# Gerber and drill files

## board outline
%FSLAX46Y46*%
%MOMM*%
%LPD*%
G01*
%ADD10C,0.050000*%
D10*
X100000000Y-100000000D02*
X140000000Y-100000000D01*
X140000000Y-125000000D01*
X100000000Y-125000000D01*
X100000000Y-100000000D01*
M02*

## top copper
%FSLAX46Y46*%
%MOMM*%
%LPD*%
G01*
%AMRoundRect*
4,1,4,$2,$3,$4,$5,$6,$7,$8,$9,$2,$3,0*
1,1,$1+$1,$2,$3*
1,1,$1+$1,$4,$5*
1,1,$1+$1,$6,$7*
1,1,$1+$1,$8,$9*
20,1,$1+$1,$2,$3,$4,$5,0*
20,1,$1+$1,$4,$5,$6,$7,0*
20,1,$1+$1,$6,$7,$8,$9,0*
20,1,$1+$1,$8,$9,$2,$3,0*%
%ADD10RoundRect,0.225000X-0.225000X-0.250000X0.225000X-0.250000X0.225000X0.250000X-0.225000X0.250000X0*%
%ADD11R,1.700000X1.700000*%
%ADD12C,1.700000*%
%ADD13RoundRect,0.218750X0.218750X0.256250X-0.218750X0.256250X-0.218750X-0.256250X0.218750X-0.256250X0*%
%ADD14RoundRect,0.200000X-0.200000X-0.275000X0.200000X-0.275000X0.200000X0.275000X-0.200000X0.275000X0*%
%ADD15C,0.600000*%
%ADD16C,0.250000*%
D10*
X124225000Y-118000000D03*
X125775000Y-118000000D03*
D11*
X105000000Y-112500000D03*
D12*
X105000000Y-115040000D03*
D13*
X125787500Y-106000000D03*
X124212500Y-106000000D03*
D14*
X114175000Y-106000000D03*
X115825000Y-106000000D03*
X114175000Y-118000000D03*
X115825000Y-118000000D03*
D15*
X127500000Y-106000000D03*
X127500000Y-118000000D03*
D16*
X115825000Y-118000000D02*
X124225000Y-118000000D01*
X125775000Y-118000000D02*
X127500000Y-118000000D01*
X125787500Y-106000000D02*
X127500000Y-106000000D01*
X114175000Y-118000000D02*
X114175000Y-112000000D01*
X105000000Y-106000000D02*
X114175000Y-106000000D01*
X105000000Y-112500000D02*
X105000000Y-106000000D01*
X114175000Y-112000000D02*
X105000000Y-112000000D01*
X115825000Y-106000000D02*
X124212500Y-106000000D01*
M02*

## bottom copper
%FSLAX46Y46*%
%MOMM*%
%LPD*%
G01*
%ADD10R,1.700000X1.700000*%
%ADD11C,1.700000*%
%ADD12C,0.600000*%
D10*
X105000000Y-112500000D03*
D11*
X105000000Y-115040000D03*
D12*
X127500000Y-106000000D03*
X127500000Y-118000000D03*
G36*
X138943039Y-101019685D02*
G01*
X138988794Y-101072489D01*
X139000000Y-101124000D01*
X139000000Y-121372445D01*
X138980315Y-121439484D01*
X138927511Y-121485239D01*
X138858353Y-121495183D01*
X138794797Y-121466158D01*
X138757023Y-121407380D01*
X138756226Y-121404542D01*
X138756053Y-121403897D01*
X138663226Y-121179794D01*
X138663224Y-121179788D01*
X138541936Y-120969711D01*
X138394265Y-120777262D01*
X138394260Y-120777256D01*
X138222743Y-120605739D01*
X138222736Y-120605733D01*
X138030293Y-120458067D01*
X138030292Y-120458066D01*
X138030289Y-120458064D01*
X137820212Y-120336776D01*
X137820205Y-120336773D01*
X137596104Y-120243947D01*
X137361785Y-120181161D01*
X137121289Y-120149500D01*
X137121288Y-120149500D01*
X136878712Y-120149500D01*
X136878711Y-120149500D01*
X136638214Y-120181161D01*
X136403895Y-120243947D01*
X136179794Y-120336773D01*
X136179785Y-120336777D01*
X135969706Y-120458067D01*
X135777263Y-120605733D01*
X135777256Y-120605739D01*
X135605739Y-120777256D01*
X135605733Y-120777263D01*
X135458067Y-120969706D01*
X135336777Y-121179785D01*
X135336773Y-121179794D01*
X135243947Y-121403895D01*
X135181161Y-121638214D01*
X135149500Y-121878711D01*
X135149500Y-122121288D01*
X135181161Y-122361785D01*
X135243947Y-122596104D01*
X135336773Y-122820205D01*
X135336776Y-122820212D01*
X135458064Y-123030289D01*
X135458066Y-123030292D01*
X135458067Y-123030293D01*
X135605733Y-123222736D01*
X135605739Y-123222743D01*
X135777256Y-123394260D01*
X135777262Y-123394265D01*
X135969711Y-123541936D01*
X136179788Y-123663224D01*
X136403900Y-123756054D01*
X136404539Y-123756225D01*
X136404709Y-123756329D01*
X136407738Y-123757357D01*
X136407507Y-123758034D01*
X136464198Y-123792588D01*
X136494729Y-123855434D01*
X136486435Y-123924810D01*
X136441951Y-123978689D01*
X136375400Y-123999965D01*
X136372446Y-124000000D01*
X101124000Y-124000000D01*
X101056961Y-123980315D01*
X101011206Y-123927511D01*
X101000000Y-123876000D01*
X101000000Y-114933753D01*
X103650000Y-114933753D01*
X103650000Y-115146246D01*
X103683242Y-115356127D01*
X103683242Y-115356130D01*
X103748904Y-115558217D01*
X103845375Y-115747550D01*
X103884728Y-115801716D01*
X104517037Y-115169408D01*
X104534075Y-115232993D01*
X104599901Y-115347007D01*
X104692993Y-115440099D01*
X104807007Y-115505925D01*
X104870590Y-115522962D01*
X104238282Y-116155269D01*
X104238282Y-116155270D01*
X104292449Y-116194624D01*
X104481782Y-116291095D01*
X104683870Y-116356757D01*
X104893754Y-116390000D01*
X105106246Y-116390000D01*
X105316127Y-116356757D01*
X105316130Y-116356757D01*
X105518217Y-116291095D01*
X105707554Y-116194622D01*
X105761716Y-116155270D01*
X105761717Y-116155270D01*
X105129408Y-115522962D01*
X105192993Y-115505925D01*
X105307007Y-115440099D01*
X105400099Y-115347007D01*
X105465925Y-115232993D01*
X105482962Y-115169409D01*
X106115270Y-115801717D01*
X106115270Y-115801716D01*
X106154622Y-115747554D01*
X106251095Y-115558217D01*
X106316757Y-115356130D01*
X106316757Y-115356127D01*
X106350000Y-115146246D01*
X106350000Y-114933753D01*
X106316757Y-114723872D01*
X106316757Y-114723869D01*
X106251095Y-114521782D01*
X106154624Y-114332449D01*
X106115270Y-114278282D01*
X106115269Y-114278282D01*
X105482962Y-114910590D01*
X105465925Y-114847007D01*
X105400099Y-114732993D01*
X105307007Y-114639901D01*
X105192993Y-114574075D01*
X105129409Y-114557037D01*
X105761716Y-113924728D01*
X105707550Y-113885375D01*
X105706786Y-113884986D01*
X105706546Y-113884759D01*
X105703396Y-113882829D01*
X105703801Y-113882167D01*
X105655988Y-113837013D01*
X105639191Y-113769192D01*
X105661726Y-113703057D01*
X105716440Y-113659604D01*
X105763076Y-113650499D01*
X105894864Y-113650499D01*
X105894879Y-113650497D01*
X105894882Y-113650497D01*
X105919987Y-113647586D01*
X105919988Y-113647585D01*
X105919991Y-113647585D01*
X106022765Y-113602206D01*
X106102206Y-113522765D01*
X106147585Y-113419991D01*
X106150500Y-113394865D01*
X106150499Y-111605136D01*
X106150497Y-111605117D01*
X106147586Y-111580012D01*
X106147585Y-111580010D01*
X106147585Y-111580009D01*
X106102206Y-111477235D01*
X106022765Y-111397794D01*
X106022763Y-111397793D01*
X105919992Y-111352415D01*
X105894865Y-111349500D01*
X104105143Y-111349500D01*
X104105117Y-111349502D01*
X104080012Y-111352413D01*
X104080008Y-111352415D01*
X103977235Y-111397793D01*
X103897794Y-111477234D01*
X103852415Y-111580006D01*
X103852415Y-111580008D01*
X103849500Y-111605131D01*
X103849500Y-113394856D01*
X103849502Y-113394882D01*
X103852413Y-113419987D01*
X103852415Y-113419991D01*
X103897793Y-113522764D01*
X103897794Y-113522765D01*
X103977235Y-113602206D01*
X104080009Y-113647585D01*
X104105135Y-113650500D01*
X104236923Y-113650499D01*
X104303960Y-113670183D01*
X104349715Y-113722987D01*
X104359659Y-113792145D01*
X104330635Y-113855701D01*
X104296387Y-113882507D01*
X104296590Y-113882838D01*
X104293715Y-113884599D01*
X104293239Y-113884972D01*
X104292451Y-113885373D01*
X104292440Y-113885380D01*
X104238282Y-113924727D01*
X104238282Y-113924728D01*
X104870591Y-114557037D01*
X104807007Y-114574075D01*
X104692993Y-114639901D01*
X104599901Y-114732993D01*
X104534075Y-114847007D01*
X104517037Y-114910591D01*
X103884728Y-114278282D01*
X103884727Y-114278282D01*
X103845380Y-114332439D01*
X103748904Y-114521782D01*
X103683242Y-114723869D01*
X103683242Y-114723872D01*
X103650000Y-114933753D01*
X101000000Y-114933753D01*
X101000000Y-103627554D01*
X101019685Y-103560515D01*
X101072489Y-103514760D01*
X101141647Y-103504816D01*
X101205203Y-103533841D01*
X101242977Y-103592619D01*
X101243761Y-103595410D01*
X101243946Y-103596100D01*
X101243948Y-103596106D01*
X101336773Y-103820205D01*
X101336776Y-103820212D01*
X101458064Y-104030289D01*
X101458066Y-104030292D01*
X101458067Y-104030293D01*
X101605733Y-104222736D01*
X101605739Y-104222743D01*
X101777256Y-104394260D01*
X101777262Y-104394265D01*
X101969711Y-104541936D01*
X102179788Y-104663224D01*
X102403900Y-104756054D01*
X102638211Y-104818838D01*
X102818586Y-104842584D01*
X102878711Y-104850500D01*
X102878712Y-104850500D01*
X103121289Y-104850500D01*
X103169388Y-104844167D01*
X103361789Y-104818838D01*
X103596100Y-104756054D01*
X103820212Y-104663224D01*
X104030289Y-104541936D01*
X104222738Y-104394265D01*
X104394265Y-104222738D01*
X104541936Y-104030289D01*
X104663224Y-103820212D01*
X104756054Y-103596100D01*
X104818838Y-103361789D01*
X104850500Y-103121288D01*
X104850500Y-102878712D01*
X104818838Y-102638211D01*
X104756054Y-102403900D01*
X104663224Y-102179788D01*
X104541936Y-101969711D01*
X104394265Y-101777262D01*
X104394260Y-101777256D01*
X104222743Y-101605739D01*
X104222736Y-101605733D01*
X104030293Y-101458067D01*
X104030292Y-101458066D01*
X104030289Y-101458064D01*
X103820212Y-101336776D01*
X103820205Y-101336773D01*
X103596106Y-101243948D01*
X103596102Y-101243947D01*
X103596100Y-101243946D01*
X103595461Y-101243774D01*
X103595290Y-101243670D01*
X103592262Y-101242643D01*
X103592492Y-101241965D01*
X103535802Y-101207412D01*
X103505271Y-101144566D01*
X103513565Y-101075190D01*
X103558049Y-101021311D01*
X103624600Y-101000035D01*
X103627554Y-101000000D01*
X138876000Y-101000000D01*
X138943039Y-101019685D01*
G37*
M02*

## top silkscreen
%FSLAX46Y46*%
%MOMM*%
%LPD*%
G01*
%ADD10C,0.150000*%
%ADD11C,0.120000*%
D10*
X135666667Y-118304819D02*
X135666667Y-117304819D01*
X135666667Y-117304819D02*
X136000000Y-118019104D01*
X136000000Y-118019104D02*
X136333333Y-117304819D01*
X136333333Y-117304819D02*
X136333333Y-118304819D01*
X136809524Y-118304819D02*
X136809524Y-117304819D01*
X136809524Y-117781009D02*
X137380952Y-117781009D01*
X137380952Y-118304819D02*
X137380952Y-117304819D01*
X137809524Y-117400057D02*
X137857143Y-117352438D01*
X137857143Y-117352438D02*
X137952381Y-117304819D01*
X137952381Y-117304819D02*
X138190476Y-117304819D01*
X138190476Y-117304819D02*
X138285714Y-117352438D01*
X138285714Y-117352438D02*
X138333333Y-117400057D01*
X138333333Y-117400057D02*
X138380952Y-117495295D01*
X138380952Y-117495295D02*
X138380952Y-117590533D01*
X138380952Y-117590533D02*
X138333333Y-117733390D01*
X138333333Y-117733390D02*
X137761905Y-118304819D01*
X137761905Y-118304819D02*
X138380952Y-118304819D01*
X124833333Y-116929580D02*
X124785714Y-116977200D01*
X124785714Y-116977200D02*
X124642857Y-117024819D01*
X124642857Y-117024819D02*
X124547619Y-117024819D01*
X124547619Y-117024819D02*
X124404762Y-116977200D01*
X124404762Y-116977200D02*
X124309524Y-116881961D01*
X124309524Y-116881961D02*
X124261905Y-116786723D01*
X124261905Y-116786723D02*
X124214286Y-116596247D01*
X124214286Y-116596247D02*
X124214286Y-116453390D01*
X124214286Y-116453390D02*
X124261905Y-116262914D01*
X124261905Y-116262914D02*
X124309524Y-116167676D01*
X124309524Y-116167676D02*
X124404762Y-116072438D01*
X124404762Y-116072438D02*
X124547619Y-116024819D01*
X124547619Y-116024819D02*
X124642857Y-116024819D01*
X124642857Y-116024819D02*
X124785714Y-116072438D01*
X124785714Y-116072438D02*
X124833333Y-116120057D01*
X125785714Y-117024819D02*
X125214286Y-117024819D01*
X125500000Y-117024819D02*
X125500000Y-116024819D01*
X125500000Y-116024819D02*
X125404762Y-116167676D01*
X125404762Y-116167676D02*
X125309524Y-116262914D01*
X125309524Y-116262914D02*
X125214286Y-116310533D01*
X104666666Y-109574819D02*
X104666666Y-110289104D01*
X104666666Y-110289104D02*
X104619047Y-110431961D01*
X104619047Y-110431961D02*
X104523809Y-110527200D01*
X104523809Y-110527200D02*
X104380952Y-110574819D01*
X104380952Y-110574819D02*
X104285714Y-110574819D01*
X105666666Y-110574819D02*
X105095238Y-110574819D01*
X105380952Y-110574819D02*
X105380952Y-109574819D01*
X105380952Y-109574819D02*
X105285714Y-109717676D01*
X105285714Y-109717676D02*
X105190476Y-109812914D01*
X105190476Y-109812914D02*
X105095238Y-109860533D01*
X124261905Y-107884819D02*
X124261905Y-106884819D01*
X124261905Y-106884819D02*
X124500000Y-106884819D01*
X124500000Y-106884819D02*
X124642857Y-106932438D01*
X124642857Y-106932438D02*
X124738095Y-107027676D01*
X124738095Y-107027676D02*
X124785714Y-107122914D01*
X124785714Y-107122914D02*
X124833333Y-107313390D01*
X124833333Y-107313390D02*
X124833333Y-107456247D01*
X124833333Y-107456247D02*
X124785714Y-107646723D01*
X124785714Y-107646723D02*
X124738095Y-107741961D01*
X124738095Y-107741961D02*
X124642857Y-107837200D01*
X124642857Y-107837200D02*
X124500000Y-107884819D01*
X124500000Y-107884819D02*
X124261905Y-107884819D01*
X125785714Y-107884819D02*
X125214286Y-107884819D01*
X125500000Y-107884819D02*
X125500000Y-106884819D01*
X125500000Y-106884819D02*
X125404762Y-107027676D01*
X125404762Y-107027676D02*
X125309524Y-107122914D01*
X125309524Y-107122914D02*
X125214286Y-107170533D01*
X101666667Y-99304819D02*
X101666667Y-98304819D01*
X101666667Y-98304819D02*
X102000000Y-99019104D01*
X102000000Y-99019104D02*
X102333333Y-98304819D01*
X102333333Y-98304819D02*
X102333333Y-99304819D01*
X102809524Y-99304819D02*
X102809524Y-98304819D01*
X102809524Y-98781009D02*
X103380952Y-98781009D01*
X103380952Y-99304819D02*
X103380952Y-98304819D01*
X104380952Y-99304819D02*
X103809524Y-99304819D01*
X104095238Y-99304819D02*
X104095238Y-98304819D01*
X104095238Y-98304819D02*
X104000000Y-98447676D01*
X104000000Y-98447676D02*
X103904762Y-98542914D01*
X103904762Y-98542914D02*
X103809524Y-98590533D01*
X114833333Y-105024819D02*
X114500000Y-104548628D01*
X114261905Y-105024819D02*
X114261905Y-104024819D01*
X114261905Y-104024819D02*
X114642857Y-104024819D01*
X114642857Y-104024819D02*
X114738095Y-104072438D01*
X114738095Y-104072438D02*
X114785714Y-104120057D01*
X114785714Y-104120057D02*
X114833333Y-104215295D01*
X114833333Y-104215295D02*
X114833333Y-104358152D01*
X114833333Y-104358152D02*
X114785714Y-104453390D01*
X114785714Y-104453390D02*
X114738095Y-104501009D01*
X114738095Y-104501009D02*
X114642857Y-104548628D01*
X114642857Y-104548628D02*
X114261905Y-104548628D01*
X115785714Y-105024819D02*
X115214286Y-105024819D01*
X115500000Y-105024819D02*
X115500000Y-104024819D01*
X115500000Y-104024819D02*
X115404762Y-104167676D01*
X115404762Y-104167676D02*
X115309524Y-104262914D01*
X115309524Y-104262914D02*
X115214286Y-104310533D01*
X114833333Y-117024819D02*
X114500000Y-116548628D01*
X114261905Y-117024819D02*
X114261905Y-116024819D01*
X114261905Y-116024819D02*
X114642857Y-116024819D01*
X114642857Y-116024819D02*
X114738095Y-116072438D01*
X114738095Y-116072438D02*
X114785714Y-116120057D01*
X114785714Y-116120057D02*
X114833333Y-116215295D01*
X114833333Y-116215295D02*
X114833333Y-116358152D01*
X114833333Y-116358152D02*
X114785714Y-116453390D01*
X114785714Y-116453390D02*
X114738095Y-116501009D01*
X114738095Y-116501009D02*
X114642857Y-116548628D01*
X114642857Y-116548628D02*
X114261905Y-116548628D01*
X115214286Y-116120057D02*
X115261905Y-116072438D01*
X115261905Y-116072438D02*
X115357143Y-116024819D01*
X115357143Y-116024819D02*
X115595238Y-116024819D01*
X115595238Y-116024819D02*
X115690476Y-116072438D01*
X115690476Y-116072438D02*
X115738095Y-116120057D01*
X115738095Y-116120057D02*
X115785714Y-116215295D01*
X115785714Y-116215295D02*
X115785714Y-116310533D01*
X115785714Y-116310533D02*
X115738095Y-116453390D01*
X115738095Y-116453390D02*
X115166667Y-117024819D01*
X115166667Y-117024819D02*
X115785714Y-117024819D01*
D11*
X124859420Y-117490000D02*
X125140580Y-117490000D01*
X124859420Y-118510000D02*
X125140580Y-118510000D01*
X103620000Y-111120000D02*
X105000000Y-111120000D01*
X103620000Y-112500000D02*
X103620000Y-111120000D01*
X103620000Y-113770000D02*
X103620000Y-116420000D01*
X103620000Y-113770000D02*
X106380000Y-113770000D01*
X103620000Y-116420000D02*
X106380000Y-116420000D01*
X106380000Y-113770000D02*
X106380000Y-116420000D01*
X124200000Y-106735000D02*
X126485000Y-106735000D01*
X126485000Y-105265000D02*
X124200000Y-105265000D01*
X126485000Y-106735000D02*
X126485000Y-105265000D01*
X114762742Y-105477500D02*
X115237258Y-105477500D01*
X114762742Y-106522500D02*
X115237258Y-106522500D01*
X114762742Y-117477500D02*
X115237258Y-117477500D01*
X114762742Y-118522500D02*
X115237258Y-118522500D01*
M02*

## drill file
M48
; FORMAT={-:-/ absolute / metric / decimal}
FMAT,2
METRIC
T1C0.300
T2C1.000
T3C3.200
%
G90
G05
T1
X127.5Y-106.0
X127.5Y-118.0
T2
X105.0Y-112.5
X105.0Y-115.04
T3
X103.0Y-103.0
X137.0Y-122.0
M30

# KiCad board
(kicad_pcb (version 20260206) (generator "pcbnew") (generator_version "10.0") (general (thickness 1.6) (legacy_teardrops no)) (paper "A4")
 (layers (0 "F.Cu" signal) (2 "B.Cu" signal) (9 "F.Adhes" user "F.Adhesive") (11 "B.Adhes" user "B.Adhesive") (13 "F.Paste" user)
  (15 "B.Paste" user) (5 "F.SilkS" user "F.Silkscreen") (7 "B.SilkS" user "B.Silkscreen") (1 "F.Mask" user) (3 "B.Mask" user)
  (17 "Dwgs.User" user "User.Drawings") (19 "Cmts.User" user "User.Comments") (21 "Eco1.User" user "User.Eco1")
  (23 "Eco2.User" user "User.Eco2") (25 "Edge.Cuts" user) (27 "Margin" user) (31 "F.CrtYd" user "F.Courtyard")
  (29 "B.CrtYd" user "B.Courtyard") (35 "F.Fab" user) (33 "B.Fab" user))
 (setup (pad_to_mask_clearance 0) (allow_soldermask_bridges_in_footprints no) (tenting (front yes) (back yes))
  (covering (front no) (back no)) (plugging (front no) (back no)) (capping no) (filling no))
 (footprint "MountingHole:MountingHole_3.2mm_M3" (layer "F.Cu") (at 137 122)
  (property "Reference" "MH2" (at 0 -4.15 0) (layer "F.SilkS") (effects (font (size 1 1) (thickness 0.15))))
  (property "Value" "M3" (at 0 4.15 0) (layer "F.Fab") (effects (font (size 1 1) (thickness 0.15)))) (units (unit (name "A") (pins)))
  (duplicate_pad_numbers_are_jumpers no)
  (pad "" np_thru_hole circle (at 0 0) (size 3.2 3.2) (drill 3.2) (layers "*.Cu" "*.Mask")))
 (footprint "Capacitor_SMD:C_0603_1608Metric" (layer "F.Cu") (at 125 118)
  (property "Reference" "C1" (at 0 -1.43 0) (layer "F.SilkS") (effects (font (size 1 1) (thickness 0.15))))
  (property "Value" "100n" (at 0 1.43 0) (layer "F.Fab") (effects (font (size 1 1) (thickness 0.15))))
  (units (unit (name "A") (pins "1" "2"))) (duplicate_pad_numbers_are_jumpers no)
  (fp_line (start -0.14058 -0.51) (end 0.14058 -0.51) (stroke (width 0.12) (type solid)) (layer "F.SilkS"))
  (fp_line (start -0.14058 0.51) (end 0.14058 0.51) (stroke (width 0.12) (type solid)) (layer "F.SilkS"))
  (pad "1" smd roundrect (at -0.775 0) (size 0.9 0.95) (layers "F.Cu" "F.Mask" "F.Paste") (roundrect_rratio 0.25) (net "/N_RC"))
  (pad "2" smd roundrect (at 0.775 0) (size 0.9 0.95) (layers "F.Cu" "F.Mask" "F.Paste") (roundrect_rratio 0.25) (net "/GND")))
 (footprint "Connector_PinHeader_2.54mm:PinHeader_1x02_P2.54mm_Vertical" (layer "F.Cu") (at 105 112.5)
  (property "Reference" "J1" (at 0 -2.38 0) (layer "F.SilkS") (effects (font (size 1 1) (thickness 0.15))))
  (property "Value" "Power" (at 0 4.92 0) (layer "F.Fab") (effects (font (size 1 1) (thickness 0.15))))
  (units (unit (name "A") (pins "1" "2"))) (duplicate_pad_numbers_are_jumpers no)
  (fp_line (start -1.38 -1.38) (end 0 -1.38) (stroke (width 0.12) (type solid)) (layer "F.SilkS"))
  (fp_line (start -1.38 0) (end -1.38 -1.38) (stroke (width 0.12) (type solid)) (layer "F.SilkS"))
  (fp_line (start -1.38 1.27) (end -1.38 3.92) (stroke (width 0.12) (type solid)) (layer "F.SilkS"))
  (fp_line (start -1.38 1.27) (end 1.38 1.27) (stroke (width 0.12) (type solid)) (layer "F.SilkS"))
  (fp_line (start -1.38 3.92) (end 1.38 3.92) (stroke (width 0.12) (type solid)) (layer "F.SilkS"))
  (fp_line (start 1.38 1.27) (end 1.38 3.92) (stroke (width 0.12) (type solid)) (layer "F.SilkS"))
  (pad "1" thru_hole rect (at 0 0) (size 1.7 1.7) (drill 1) (layers "*.Cu" "*.Mask") (remove_unused_layers no) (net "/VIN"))
  (pad "2" thru_hole circle (at 0 2.54) (size 1.7 1.7) (drill 1) (layers "*.Cu" "*.Mask") (remove_unused_layers no) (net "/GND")))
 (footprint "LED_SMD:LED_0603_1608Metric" (layer "F.Cu") (at 125 106 180)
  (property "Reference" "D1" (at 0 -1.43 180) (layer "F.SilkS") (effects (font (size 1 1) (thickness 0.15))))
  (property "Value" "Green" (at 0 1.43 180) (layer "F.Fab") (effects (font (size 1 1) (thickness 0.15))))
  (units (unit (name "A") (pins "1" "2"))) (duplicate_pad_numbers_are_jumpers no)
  (fp_line (start 0.8 -0.735) (end -1.485 -0.735) (stroke (width 0.12) (type solid)) (layer "F.SilkS"))
  (fp_line (start -1.485 0.735) (end 0.8 0.735) (stroke (width 0.12) (type solid)) (layer "F.SilkS"))
  (fp_line (start -1.485 -0.735) (end -1.485 0.735) (stroke (width 0.12) (type solid)) (layer "F.SilkS"))
  (pad "1" smd roundrect (at -0.7875 0 180) (size 0.875 0.95) (layers "F.Cu" "F.Mask" "F.Paste") (roundrect_rratio 0.25) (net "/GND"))
  (pad "2" smd roundrect (at 0.7875 0 180) (size 0.875 0.95) (layers "F.Cu" "F.Mask" "F.Paste") (roundrect_rratio 0.25) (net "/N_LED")))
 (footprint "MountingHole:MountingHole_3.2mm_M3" (layer "F.Cu") (at 103 103)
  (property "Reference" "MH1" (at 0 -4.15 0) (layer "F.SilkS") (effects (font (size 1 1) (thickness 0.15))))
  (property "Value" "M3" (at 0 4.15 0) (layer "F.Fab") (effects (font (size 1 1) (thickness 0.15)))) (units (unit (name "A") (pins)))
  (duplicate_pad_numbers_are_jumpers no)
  (pad "" np_thru_hole circle (at 0 0) (size 3.2 3.2) (drill 3.2) (layers "*.Cu" "*.Mask")))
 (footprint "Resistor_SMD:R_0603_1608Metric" (layer "F.Cu") (at 115 106)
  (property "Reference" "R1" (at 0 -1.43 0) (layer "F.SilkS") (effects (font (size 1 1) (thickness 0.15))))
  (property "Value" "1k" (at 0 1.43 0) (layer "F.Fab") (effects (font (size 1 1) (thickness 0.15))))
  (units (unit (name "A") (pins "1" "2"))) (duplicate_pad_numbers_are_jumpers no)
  (fp_line (start -0.237258 -0.5225) (end 0.237258 -0.5225) (stroke (width 0.12) (type solid)) (layer "F.SilkS"))
  (fp_line (start -0.237258 0.5225) (end 0.237258 0.5225) (stroke (width 0.12) (type solid)) (layer "F.SilkS"))
  (pad "1" smd roundrect (at -0.825 0) (size 0.8 0.95) (layers "F.Cu" "F.Mask" "F.Paste") (roundrect_rratio 0.25) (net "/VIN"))
  (pad "2" smd roundrect (at 0.825 0) (size 0.8 0.95) (layers "F.Cu" "F.Mask" "F.Paste") (roundrect_rratio 0.25) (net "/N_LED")))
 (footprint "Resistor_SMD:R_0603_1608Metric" (layer "F.Cu") (at 115 118)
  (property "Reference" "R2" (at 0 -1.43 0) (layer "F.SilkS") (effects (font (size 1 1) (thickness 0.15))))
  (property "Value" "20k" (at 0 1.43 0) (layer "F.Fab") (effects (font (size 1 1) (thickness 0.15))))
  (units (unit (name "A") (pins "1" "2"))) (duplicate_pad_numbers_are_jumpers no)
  (fp_line (start -0.237258 -0.5225) (end 0.237258 -0.5225) (stroke (width 0.12) (type solid)) (layer "F.SilkS"))
  (fp_line (start -0.237258 0.5225) (end 0.237258 0.5225) (stroke (width 0.12) (type solid)) (layer "F.SilkS"))
  (pad "1" smd roundrect (at -0.825 0) (size 0.8 0.95) (layers "F.Cu" "F.Mask" "F.Paste") (roundrect_rratio 0.25) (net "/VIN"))
  (pad "2" smd roundrect (at 0.825 0) (size 0.8 0.95) (layers "F.Cu" "F.Mask" "F.Paste") (roundrect_rratio 0.25) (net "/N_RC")))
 (gr_rect (start 100 100) (end 140 125) (stroke (width 0.05) (type default)) (fill no) (layer "Edge.Cuts"))
 (segment (start 115.825 118) (end 124.225 118) (width 0.25) (layer "F.Cu") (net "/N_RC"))
 (segment (start 125.775 118) (end 127.5 118) (width 0.25) (layer "F.Cu") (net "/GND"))
 (segment (start 125.7875 106) (end 127.5 106) (width 0.25) (layer "F.Cu") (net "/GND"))
 (via (at 127.5 106) (size 0.6) (drill 0.3) (layers "F.Cu" "B.Cu") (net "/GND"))
 (via (at 127.5 118) (size 0.6) (drill 0.3) (layers "F.Cu" "B.Cu") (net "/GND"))
 (segment (start 114.175 118) (end 114.175 112) (width 0.25) (layer "F.Cu") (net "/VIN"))
 (segment (start 105 106) (end 114.175 106) (width 0.25) (layer "F.Cu") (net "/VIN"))
 (segment (start 105 112.5) (end 105 106) (width 0.25) (layer "F.Cu") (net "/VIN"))
 (segment (start 114.175 112) (end 105 112) (width 0.25) (layer "F.Cu") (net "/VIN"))
 (segment (start 115.825 106) (end 124.2125 106) (width 0.25) (layer "F.Cu") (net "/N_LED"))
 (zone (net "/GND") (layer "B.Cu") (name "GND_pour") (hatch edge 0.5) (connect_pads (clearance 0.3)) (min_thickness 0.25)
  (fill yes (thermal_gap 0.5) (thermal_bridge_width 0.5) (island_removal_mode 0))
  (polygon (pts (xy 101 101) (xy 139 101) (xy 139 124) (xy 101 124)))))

